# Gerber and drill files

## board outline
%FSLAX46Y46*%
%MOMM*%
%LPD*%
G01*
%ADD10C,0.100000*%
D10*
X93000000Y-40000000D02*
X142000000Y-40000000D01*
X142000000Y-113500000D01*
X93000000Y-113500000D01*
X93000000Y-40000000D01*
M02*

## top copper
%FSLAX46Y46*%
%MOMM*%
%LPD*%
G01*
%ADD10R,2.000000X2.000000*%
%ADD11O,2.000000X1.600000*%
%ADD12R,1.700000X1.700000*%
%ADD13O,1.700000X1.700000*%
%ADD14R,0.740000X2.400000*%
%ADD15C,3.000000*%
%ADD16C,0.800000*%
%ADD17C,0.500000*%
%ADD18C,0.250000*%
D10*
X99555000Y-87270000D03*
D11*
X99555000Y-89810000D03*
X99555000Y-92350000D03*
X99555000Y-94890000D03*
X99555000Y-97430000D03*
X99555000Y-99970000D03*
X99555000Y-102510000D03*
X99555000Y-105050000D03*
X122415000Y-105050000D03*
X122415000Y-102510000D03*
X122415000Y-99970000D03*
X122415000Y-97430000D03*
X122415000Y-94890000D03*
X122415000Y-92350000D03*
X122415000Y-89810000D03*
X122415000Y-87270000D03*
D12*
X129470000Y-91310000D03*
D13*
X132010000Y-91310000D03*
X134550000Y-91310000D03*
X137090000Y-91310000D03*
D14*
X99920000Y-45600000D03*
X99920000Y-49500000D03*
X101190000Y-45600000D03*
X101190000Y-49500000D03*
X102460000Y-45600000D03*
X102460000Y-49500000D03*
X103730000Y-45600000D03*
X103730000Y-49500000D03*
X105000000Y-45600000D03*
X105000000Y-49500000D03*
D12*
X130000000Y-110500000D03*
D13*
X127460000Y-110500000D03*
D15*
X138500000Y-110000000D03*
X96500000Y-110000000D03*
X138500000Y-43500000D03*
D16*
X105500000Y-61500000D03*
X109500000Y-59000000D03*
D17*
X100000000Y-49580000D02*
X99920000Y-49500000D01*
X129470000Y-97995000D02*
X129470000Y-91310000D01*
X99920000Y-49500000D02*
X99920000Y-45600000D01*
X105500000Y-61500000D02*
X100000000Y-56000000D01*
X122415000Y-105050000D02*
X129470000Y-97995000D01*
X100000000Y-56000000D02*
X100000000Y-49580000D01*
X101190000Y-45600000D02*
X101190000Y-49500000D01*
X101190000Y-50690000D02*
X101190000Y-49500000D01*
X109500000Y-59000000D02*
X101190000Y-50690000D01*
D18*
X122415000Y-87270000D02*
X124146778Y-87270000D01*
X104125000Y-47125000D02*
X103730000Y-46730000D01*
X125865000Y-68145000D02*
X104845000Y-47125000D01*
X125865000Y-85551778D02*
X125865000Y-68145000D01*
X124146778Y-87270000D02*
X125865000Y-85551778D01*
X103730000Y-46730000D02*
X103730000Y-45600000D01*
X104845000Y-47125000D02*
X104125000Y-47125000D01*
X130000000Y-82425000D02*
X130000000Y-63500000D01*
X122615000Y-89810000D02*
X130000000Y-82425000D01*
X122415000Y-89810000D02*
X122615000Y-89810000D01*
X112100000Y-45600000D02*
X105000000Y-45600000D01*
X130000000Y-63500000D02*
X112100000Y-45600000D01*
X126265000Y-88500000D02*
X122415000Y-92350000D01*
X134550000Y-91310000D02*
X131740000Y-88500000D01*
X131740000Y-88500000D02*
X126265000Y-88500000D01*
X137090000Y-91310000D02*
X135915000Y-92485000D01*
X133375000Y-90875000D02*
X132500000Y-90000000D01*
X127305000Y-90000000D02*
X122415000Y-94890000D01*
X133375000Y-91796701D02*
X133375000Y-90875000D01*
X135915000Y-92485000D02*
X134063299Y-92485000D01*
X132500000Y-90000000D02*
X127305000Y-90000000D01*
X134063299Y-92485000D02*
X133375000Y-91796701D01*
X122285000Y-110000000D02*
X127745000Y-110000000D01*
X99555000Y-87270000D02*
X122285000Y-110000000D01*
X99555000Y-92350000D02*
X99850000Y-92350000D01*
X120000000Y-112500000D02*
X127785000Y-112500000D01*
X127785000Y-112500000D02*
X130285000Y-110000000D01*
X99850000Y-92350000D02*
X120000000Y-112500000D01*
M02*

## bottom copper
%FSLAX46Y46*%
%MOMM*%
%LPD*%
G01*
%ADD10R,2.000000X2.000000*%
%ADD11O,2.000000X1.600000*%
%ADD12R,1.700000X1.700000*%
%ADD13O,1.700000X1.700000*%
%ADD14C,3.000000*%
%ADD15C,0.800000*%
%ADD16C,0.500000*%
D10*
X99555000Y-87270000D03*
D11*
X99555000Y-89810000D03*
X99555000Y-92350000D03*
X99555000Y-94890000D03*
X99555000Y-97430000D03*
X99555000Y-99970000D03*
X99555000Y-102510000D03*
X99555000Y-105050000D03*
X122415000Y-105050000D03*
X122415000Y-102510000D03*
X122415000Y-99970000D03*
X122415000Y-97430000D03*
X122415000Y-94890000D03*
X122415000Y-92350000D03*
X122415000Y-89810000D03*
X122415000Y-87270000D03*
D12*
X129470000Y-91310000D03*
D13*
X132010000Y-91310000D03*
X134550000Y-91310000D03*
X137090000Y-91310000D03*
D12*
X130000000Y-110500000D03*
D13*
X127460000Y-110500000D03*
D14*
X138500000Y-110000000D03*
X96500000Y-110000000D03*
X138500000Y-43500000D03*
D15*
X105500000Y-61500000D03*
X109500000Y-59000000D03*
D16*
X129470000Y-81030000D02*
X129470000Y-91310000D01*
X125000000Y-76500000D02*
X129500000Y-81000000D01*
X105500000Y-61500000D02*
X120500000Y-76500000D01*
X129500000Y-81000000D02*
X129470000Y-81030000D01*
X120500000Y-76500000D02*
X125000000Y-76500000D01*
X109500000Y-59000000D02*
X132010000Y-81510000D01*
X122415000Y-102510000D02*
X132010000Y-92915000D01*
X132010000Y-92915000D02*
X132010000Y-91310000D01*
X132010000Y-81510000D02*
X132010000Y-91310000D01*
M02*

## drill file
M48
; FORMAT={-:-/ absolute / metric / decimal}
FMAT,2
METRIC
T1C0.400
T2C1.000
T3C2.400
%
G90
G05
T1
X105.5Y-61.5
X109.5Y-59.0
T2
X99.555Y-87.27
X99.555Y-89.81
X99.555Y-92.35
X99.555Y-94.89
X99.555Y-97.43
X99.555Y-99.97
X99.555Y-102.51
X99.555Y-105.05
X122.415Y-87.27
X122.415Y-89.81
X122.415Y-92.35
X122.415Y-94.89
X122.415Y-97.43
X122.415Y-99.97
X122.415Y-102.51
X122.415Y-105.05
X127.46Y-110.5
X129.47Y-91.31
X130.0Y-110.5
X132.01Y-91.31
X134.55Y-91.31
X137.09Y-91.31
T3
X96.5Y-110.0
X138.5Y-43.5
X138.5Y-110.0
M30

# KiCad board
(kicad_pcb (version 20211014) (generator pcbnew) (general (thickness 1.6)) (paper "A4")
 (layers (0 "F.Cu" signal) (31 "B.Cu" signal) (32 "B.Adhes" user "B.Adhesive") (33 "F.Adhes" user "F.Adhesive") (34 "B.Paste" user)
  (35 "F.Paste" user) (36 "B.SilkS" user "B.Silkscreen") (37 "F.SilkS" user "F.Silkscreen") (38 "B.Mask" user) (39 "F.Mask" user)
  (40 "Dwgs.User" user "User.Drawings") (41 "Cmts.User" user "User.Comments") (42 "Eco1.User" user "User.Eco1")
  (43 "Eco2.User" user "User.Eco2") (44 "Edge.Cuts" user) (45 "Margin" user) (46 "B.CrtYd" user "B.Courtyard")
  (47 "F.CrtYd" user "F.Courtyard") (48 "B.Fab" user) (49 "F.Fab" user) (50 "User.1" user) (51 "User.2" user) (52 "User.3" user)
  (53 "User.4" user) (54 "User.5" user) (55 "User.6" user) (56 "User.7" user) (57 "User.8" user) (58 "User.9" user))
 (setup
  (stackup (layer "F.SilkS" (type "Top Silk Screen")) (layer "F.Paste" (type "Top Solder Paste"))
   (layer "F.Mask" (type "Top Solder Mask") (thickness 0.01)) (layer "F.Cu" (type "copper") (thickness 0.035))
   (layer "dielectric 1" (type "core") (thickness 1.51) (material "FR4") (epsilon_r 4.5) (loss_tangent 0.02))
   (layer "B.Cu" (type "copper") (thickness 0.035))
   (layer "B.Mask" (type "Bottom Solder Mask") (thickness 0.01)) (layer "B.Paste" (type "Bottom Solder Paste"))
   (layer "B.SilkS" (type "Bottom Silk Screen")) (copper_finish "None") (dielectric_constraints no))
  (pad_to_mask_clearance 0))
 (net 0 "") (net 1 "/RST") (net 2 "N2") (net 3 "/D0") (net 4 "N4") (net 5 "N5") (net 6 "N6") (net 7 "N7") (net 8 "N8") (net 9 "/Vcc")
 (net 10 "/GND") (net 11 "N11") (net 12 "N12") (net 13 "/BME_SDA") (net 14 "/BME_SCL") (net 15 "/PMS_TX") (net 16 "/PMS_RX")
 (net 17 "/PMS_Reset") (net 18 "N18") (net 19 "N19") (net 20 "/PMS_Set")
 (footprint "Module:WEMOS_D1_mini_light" (layer "F.Cu") (at 99.555 87.27)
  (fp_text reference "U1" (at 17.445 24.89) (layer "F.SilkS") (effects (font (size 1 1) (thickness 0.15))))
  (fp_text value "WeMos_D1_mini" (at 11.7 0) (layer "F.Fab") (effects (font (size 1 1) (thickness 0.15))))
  (pad "1" thru_hole rect (at 0 0) (size 2 2) (drill 1) (layers *.Cu *.Mask) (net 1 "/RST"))
  (pad "2" thru_hole oval (at 0 2.54) (size 2 1.6) (drill 1) (layers *.Cu *.Mask) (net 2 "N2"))
  (pad "3" thru_hole oval (at 0 5.08) (size 2 1.6) (drill 1) (layers *.Cu *.Mask) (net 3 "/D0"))
  (pad "4" thru_hole oval (at 0 7.62) (size 2 1.6) (drill 1) (layers *.Cu *.Mask) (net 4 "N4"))
  (pad "5" thru_hole oval (at 0 10.16) (size 2 1.6) (drill 1) (layers *.Cu *.Mask) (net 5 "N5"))
  (pad "6" thru_hole oval (at 0 12.7) (size 2 1.6) (drill 1) (layers *.Cu *.Mask) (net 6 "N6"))
  (pad "7" thru_hole oval (at 0 15.24) (size 2 1.6) (drill 1) (layers *.Cu *.Mask) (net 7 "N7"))
  (pad "8" thru_hole oval (at 0 17.78) (size 2 1.6) (drill 1) (layers *.Cu *.Mask) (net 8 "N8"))
  (pad "9" thru_hole oval (at 22.86 17.78) (size 2 1.6) (drill 1) (layers *.Cu *.Mask) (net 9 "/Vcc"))
  (pad "10" thru_hole oval (at 22.86 15.24) (size 2 1.6) (drill 1) (layers *.Cu *.Mask) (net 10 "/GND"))
  (pad "11" thru_hole oval (at 22.86 12.7) (size 2 1.6) (drill 1) (layers *.Cu *.Mask) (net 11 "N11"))
  (pad "12" thru_hole oval (at 22.86 10.16) (size 2 1.6) (drill 1) (layers *.Cu *.Mask) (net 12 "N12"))
  (pad "13" thru_hole oval (at 22.86 7.62) (size 2 1.6) (drill 1) (layers *.Cu *.Mask) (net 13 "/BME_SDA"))
  (pad "14" thru_hole oval (at 22.86 5.08) (size 2 1.6) (drill 1) (layers *.Cu *.Mask) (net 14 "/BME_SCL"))
  (pad "15" thru_hole oval (at 22.86 2.54) (size 2 1.6) (drill 1) (layers *.Cu *.Mask) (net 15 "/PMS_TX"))
  (pad "16" thru_hole oval (at 22.86 0) (size 2 1.6) (drill 1) (layers *.Cu *.Mask) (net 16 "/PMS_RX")))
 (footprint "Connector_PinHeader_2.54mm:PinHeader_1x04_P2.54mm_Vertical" (layer "F.Cu") (at 129.47 91.31 90)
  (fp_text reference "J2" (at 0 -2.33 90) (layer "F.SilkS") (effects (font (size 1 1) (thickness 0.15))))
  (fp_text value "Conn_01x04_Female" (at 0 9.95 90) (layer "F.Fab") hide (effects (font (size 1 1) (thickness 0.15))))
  (pad "1" thru_hole rect (at 0 0 90) (size 1.7 1.7) (drill 1) (layers *.Cu *.Mask) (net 9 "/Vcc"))
  (pad "2" thru_hole oval (at 0 2.54 90) (size 1.7 1.7) (drill 1) (layers *.Cu *.Mask) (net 10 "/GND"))
  (pad "3" thru_hole oval (at 0 5.08 90) (size 1.7 1.7) (drill 1) (layers *.Cu *.Mask) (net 14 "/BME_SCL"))
  (pad "4" thru_hole oval (at 0 7.62 90) (size 1.7 1.7) (drill 1) (layers *.Cu *.Mask) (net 13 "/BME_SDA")))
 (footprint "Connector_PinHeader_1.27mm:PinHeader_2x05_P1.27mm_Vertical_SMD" (layer "F.Cu") (at 102.46 47.55 90)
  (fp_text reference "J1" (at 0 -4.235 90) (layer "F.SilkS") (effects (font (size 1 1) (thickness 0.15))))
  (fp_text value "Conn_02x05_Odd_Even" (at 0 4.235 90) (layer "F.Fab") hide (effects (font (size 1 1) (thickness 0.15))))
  (pad "1" smd rect (at 1.95 -2.54 90) (size 2.4 0.74) (layers "F.Cu" "F.Paste" "F.Mask") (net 9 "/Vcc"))
  (pad "2" smd rect (at -1.95 -2.54 90) (size 2.4 0.74) (layers "F.Cu" "F.Paste" "F.Mask") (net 9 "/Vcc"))
  (pad "3" smd rect (at 1.95 -1.27 90) (size 2.4 0.74) (layers "F.Cu" "F.Paste" "F.Mask") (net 10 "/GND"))
  (pad "4" smd rect (at -1.95 -1.27 90) (size 2.4 0.74) (layers "F.Cu" "F.Paste" "F.Mask") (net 10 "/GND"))
  (pad "5" smd rect (at 1.95 0 90) (size 2.4 0.74) (layers "F.Cu" "F.Paste" "F.Mask") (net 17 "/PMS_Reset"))
  (pad "6" smd rect (at -1.95 0 90) (size 2.4 0.74) (layers "F.Cu" "F.Paste" "F.Mask") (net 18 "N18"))
  (pad "7" smd rect (at 1.95 1.27 90) (size 2.4 0.74) (layers "F.Cu" "F.Paste" "F.Mask") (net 16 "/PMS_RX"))
  (pad "8" smd rect (at -1.95 1.27 90) (size 2.4 0.74) (layers "F.Cu" "F.Paste" "F.Mask") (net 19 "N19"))
  (pad "9" smd rect (at 1.95 2.54 90) (size 2.4 0.74) (layers "F.Cu" "F.Paste" "F.Mask") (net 15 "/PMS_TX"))
  (pad "10" smd rect (at -1.95 2.54 90) (size 2.4 0.74) (layers "F.Cu" "F.Paste" "F.Mask") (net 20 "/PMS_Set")))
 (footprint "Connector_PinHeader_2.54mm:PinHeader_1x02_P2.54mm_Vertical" (layer "F.Cu") (at 130 110.5 -90)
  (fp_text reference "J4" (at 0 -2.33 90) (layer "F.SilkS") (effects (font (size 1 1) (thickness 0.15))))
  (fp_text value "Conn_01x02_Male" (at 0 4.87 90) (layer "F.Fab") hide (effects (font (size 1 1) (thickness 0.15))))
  (pad "1" thru_hole rect (at 0 0 270) (size 1.7 1.7) (drill 1) (layers *.Cu *.Mask) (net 3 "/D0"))
  (pad "2" thru_hole oval (at 0 2.54 270) (size 1.7 1.7) (drill 1) (layers *.Cu *.Mask) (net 1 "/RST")))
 (gr_rect (start 93 40) (end 142 113.5) (layer "Edge.Cuts") (width 0.1) (fill none))
 (via (at 138.5 110) (size 3) (drill 2.4) (layers "F.Cu" "B.Cu") (free) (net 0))
 (via (at 96.5 110) (size 3) (drill 2.4) (layers "F.Cu" "B.Cu") (free) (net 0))
 (via (at 138.5 43.5) (size 3) (drill 2.4) (layers "F.Cu" "B.Cu") (free) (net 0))
 (segment (start 100 49.58) (end 99.92 49.5) (width 0.5) (layer "F.Cu") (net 9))
 (segment (start 129.47 97.995) (end 129.47 91.31) (width 0.5) (layer "F.Cu") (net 9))
 (segment (start 99.92 49.5) (end 99.92 45.6) (width 0.5) (layer "F.Cu") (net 9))
 (segment (start 105.5 61.5) (end 100 56) (width 0.5) (layer "F.Cu") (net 9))
 (segment (start 122.415 105.05) (end 129.47 97.995) (width 0.5) (layer "F.Cu") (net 9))
 (segment (start 100 56) (end 100 49.58) (width 0.5) (layer "F.Cu") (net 9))
 (via (at 105.5 61.5) (size 0.8) (drill 0.4) (layers "F.Cu" "B.Cu") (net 9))
 (segment (start 129.47 81.03) (end 129.47 91.31) (width 0.5) (layer "B.Cu") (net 9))
 (segment (start 125 76.5) (end 129.5 81) (width 0.5) (layer "B.Cu") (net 9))
 (segment (start 105.5 61.5) (end 120.5 76.5) (width 0.5) (layer "B.Cu") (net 9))
 (segment (start 129.5 81) (end 129.47 81.03) (width 0.5) (layer "B.Cu") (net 9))
 (segment (start 120.5 76.5) (end 125 76.5) (width 0.5) (layer "B.Cu") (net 9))
 (segment (start 101.19 45.6) (end 101.19 49.5) (width 0.5) (layer "F.Cu") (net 10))
 (segment (start 101.19 50.69) (end 101.19 49.5) (width 0.5) (layer "F.Cu") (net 10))
 (segment (start 109.5 59) (end 101.19 50.69) (width 0.5) (layer "F.Cu") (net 10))
 (via (at 109.5 59) (size 0.8) (drill 0.4) (layers "F.Cu" "B.Cu") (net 10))
 (segment (start 109.5 59) (end 132.01 81.51) (width 0.5) (layer "B.Cu") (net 10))
 (segment (start 122.415 102.51) (end 132.01 92.915) (width 0.5) (layer "B.Cu") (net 10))
 (segment (start 132.01 92.915) (end 132.01 91.31) (width 0.5) (layer "B.Cu") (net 10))
 (segment (start 132.01 81.51) (end 132.01 91.31) (width 0.5) (layer "B.Cu") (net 10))
 (segment (start 122.415 87.27) (end 124.146778 87.27) (width 0.25) (layer "F.Cu") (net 16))
 (segment (start 104.125 47.125) (end 103.73 46.73) (width 0.25) (layer "F.Cu") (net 16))
 (segment (start 125.865 68.145) (end 104.845 47.125) (width 0.25) (layer "F.Cu") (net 16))
 (segment (start 125.865 85.551778) (end 125.865 68.145) (width 0.25) (layer "F.Cu") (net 16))
 (segment (start 124.146778 87.27) (end 125.865 85.551778) (width 0.25) (layer "F.Cu") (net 16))
 (segment (start 103.73 46.73) (end 103.73 45.6) (width 0.25) (layer "F.Cu") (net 16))
 (segment (start 104.845 47.125) (end 104.125 47.125) (width 0.25) (layer "F.Cu") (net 16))
 (segment (start 130 82.425) (end 130 63.5) (width 0.25) (layer "F.Cu") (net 15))
 (segment (start 122.615 89.81) (end 130 82.425) (width 0.25) (layer "F.Cu") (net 15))
 (segment (start 122.415 89.81) (end 122.615 89.81) (width 0.25) (layer "F.Cu") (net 15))
 (segment (start 112.1 45.6) (end 105 45.6) (width 0.25) (layer "F.Cu") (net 15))
 (segment (start 130 63.5) (end 112.1 45.6) (width 0.25) (layer "F.Cu") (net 15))
 (segment (start 126.265 88.5) (end 122.415 92.35) (width 0.25) (layer "F.Cu") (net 14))
 (segment (start 134.55 91.31) (end 131.74 88.5) (width 0.25) (layer "F.Cu") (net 14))
 (segment (start 131.74 88.5) (end 126.265 88.5) (width 0.25) (layer "F.Cu") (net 14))
 (segment (start 137.09 91.31) (end 135.915 92.485) (width 0.25) (layer "F.Cu") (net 13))
 (segment (start 133.375 90.875) (end 132.5 90) (width 0.25) (layer "F.Cu") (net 13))
 (segment (start 127.305 90) (end 122.415 94.89) (width 0.25) (layer "F.Cu") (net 13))
 (segment (start 133.375 91.796701) (end 133.375 90.875) (width 0.25) (layer "F.Cu") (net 13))
 (segment (start 135.915 92.485) (end 134.063299 92.485) (width 0.25) (layer "F.Cu") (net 13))
 (segment (start 132.5 90) (end 127.305 90) (width 0.25) (layer "F.Cu") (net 13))
 (segment (start 134.063299 92.485) (end 133.375 91.796701) (width 0.25) (layer "F.Cu") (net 13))
 (segment (start 122.285 110) (end 127.745 110) (width 0.25) (layer "F.Cu") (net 1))
 (segment (start 99.555 87.27) (end 122.285 110) (width 0.25) (layer "F.Cu") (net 1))
 (segment (start 99.555 92.35) (end 99.85 92.35) (width 0.25) (layer "F.Cu") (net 3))
 (segment (start 120 112.5) (end 127.785 112.5) (width 0.25) (layer "F.Cu") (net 3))
 (segment (start 127.785 112.5) (end 130.285 110) (width 0.25) (layer "F.Cu") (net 3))
 (segment (start 99.85 92.35) (end 120 112.5) (width 0.25) (layer "F.Cu") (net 3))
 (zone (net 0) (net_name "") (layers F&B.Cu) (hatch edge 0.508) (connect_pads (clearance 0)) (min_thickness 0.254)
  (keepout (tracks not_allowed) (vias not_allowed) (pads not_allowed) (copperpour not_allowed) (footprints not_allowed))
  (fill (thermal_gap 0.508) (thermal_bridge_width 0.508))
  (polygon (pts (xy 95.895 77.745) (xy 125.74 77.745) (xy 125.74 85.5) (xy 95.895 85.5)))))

